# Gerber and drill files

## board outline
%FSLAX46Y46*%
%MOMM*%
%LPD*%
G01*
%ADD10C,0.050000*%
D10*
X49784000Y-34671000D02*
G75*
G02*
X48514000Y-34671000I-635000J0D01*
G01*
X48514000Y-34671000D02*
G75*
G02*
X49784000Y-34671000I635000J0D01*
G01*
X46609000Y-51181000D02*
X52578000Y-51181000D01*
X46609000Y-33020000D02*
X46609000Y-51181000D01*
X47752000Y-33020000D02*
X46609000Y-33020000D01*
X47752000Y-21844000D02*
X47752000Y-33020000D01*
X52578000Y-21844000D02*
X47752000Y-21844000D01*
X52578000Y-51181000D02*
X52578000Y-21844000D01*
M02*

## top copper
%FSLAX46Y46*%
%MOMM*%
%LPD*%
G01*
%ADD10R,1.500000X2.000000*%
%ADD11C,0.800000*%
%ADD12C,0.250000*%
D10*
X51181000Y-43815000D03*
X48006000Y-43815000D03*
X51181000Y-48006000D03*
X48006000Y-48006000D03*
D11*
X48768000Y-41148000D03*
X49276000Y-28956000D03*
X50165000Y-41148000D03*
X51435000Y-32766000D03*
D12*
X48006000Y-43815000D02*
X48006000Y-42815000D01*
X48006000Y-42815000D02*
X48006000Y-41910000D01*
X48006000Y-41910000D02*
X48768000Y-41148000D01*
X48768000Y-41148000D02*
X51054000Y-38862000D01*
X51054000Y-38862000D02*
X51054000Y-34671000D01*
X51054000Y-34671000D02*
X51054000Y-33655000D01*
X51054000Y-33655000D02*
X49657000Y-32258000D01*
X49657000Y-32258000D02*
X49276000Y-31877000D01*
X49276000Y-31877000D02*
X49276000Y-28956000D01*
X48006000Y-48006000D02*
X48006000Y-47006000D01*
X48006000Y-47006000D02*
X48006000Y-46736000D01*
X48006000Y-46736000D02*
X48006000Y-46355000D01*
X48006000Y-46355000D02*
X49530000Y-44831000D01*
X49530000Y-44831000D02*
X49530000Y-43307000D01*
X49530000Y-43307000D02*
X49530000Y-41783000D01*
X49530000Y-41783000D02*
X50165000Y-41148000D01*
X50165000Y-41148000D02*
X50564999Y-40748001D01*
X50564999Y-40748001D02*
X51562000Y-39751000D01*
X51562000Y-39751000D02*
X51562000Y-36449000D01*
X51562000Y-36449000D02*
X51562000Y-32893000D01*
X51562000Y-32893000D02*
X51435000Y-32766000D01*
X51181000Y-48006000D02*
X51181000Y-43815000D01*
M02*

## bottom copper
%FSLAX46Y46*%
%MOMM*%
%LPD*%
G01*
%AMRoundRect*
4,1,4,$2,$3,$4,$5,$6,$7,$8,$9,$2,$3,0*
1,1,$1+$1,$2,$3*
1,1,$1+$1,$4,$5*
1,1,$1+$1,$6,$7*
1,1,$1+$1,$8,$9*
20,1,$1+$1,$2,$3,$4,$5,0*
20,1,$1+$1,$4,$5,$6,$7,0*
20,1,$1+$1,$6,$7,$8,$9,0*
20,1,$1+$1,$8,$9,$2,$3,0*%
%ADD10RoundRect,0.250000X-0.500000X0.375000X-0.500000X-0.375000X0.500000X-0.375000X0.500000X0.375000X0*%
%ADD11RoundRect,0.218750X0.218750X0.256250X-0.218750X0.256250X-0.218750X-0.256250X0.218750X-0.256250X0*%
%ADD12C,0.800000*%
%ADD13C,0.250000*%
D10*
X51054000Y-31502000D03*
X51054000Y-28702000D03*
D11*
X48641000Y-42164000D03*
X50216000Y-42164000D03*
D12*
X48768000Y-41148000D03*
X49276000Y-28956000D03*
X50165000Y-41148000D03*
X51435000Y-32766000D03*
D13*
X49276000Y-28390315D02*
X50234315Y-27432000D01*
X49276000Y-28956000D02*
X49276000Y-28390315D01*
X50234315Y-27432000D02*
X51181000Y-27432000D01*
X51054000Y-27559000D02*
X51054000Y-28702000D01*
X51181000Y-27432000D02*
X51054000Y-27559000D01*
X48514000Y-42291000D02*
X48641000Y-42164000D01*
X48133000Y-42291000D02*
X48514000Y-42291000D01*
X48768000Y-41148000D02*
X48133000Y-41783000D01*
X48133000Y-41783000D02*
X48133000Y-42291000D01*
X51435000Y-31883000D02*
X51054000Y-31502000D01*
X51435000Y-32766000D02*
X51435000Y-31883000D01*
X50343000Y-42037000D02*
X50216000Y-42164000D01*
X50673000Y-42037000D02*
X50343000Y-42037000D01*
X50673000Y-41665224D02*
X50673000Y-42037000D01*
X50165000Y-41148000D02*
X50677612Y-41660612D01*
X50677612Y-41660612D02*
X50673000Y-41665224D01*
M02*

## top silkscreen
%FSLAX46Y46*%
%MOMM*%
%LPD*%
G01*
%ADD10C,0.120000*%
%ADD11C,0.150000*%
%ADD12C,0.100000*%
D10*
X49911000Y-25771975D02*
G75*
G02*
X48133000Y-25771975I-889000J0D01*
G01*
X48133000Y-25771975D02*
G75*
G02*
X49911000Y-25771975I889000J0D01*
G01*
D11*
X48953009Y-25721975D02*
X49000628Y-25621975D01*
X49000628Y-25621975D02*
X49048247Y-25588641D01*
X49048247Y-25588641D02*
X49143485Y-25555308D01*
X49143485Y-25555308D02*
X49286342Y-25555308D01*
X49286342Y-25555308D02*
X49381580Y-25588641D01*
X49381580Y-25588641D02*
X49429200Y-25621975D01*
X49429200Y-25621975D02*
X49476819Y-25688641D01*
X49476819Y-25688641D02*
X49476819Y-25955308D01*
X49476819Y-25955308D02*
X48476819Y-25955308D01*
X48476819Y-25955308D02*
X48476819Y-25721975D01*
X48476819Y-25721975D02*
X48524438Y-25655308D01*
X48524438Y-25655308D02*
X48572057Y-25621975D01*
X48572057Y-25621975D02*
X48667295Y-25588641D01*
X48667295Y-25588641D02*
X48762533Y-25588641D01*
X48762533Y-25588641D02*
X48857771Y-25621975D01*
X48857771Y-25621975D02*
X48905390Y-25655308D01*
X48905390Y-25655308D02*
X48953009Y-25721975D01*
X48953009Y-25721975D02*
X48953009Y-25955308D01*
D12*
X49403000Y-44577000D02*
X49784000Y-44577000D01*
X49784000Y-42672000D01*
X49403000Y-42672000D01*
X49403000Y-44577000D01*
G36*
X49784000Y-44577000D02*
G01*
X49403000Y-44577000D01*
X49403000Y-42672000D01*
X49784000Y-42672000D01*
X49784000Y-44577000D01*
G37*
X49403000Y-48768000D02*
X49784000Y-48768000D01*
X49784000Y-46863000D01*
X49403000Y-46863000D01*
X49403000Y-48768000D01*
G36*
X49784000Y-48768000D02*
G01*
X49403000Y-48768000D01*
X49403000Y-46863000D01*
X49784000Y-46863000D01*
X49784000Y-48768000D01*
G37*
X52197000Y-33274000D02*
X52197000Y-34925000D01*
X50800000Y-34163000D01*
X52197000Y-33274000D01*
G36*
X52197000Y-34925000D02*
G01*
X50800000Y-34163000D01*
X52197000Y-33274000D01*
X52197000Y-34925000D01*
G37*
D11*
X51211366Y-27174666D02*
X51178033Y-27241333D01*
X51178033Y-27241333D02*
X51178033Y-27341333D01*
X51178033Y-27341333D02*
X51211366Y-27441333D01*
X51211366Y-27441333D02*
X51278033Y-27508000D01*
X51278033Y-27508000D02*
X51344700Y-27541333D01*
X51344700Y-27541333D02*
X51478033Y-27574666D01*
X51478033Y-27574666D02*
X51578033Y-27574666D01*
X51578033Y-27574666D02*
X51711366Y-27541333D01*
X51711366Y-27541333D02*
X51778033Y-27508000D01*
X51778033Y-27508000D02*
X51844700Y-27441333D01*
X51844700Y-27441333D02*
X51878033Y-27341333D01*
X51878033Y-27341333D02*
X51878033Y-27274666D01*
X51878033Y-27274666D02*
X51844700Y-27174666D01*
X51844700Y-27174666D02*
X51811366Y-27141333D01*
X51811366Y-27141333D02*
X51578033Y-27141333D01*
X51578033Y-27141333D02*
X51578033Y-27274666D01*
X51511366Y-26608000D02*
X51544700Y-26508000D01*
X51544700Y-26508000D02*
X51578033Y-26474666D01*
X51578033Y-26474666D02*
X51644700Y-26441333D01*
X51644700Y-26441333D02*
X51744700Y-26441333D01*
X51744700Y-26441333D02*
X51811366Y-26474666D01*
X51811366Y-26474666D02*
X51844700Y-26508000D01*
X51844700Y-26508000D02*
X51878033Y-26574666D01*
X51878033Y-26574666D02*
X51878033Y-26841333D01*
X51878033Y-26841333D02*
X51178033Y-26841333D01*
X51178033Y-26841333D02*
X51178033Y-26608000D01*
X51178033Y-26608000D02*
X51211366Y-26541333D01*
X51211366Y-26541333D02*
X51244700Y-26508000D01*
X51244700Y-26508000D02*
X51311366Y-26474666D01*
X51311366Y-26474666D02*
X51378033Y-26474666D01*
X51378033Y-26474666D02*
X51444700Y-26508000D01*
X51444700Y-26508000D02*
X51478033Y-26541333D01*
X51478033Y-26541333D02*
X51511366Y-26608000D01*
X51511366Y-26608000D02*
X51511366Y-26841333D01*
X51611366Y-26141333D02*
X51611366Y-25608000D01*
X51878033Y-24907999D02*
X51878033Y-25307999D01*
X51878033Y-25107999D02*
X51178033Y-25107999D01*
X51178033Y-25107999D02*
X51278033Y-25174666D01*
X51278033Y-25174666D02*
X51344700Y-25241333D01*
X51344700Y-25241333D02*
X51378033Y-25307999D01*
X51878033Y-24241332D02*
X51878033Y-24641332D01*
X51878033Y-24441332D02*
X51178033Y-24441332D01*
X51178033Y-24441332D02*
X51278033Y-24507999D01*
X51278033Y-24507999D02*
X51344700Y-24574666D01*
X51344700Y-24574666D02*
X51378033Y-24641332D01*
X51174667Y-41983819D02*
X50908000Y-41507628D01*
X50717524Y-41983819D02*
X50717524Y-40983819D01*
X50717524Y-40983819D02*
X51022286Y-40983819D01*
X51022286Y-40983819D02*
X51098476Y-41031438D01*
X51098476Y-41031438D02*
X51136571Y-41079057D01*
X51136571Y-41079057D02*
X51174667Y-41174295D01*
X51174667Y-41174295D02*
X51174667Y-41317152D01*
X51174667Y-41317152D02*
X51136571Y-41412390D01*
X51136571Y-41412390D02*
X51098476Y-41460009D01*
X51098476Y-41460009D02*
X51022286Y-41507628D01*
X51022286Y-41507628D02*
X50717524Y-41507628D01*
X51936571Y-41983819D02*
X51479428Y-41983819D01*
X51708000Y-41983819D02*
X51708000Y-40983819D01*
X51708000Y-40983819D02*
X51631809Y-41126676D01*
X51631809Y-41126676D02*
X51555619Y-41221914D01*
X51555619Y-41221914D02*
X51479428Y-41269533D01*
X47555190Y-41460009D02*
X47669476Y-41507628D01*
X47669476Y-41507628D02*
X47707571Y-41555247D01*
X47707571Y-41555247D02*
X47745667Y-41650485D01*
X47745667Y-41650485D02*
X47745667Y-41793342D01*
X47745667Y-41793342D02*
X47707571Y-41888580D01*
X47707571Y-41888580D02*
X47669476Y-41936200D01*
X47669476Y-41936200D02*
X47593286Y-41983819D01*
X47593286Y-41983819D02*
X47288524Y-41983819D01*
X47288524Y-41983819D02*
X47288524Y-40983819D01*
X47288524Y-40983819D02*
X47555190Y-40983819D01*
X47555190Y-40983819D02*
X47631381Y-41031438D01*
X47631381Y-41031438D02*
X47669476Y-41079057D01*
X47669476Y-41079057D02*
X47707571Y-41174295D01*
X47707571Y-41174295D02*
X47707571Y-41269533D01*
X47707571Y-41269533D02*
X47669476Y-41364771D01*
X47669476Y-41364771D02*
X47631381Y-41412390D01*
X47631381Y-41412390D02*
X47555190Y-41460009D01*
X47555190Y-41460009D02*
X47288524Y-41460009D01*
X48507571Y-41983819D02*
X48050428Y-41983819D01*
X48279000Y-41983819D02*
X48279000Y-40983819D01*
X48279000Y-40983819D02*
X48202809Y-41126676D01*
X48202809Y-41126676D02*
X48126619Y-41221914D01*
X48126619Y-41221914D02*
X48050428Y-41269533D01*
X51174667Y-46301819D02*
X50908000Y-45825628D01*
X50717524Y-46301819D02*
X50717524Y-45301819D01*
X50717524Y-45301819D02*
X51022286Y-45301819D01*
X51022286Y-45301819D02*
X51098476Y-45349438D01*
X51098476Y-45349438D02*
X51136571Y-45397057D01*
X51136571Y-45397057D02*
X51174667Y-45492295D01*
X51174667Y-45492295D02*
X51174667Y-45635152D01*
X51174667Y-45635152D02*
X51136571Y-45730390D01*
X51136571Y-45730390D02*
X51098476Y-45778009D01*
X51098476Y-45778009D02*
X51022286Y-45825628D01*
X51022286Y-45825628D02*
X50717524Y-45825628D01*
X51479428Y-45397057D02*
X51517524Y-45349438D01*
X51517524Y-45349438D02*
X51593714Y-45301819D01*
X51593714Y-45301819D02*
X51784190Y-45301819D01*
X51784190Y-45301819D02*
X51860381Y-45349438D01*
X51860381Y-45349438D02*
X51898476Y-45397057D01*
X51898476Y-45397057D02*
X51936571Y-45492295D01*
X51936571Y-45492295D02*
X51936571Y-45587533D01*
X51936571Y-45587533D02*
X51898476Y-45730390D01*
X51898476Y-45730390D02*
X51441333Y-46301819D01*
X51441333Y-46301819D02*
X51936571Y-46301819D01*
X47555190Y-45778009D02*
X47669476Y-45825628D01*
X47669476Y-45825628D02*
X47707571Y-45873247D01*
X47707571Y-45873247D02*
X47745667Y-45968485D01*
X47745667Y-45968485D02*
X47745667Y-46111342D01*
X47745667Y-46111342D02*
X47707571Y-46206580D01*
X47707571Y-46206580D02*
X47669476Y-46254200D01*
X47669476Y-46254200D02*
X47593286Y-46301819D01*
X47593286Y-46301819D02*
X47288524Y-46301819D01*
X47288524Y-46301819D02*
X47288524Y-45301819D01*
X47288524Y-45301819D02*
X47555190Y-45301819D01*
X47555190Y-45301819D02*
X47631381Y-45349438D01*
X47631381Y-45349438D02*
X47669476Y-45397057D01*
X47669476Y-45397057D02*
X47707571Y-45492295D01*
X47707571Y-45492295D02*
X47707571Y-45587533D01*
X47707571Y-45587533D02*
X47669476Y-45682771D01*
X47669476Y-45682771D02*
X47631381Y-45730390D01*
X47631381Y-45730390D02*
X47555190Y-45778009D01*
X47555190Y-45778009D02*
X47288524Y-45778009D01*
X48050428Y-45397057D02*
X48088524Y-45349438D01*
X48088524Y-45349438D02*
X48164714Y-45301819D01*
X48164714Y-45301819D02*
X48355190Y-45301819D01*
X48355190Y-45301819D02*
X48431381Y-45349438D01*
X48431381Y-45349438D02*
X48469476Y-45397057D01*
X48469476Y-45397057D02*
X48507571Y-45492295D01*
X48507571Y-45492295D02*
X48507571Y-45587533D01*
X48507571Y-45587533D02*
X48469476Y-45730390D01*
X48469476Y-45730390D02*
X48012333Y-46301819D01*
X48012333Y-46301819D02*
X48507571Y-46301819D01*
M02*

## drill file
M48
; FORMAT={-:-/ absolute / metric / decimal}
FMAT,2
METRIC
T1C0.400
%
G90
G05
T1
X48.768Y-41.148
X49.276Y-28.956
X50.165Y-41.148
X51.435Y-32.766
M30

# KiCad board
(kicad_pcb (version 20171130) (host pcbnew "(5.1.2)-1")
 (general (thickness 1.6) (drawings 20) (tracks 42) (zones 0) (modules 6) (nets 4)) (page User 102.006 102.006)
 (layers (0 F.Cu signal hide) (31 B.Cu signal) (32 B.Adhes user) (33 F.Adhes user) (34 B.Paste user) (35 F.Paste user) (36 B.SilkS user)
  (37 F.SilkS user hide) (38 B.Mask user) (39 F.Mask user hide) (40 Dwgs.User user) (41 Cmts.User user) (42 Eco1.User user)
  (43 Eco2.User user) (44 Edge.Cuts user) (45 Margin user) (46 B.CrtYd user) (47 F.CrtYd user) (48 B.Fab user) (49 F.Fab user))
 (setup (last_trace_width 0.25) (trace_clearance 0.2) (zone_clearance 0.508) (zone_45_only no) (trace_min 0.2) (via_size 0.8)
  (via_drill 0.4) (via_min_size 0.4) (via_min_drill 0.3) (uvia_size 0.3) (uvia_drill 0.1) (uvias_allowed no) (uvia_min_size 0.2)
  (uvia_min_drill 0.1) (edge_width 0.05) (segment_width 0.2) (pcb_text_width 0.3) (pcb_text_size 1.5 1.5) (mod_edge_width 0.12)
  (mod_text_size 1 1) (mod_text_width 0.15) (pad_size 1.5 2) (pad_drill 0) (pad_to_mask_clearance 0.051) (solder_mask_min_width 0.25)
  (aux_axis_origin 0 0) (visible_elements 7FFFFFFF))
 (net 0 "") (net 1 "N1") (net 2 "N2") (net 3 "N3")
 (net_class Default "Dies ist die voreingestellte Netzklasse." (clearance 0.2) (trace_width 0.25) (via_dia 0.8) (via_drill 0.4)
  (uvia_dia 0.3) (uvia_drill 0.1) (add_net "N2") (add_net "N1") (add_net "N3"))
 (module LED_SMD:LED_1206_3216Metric (layer B.Cu) (at 51.054 30.102 270)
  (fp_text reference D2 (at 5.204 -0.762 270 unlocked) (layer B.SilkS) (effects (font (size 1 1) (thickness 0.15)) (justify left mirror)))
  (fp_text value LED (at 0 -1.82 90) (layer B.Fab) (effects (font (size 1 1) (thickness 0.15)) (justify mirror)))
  (pad 2 smd roundrect (at 1.4 0 270) (size 1.25 1.5) (layers B.Cu B.Paste B.Mask) (roundrect_rratio 0.2) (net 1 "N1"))
  (pad 1 smd roundrect (at -1.4 0 270) (size 1.25 1.5) (layers B.Cu B.Paste B.Mask) (roundrect_rratio 0.2) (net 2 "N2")))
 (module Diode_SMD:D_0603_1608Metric (layer B.Cu) (at 49.4285 42.164 180)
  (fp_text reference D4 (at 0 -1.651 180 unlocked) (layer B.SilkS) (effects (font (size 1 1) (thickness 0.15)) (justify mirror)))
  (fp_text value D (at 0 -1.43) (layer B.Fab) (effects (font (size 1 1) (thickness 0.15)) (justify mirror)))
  (pad 2 smd roundrect (at 0.7875 0 180) (size 0.875 0.95) (layers B.Cu B.Paste B.Mask) (roundrect_rratio 0.25) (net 2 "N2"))
  (pad 1 smd roundrect (at -0.7875 0 180) (size 0.875 0.95) (layers B.Cu B.Paste B.Mask) (roundrect_rratio 0.25) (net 1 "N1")))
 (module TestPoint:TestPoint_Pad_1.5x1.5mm (layer F.Cu) (at 51.181 43.815)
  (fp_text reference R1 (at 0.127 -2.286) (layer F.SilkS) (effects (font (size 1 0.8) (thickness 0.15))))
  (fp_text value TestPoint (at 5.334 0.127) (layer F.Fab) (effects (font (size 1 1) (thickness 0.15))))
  (pad 1 smd rect (at 0 0) (size 1.5 2) (layers F.Cu F.Mask) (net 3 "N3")))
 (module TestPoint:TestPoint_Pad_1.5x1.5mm (layer F.Cu) (at 48.006 43.815)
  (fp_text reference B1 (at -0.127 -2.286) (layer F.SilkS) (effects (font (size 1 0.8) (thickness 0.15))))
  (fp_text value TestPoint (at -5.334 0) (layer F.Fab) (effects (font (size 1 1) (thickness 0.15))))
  (pad 1 smd rect (at 0 0) (size 1.5 2) (layers F.Cu F.Mask) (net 2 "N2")))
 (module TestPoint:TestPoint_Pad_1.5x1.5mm (layer F.Cu) (at 51.181 48.006)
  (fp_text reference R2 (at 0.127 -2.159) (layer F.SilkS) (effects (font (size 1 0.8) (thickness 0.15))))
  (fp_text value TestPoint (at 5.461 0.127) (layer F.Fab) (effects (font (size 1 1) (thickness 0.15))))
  (pad 1 smd rect (at 0 0) (size 1.5 2) (layers F.Cu F.Mask) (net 3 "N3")))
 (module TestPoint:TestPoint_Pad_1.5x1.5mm (layer F.Cu) (at 48.006 48.006)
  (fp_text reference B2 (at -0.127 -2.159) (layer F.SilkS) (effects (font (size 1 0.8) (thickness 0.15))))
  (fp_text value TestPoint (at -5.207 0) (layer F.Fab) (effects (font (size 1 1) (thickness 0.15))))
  (pad 1 smd rect (at 0 0) (size 1.5 2) (layers F.Cu F.Mask) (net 1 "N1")))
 (gr_circle (center 49.022 25.771975) (end 49.022 24.882975) (layer F.SilkS) (width 0.12))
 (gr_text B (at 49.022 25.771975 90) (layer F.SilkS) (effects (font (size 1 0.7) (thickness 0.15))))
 (gr_poly (pts (xy 49.403 44.577) (xy 49.784 44.577) (xy 49.784 42.672) (xy 49.403 42.672)) (layer F.SilkS) (width 0.1))
 (gr_poly (pts (xy 49.403 48.768) (xy 49.784 48.768) (xy 49.784 46.863) (xy 49.403 46.863)) (layer F.SilkS) (width 0.1))
 (gr_circle (center 49.149 34.671) (end 49.149 34.036) (layer Edge.Cuts) (width 0.05))
 (gr_poly (pts (xy 52.197 33.274) (xy 52.197 34.925) (xy 50.8 34.163)) (layer F.SilkS) (width 0.1))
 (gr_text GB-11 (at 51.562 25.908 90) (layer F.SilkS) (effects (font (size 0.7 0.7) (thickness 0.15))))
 (gr_line (start 46.609 51.181) (end 52.578 51.181) (layer Edge.Cuts) (width 0.05))
 (gr_line (start 46.609 33.02) (end 46.609 51.181) (layer Edge.Cuts) (width 0.05))
 (gr_line (start 47.752 33.02) (end 46.609 33.02) (layer Edge.Cuts) (width 0.05))
 (gr_line (start 47.752 21.844) (end 47.752 33.02) (layer Edge.Cuts) (width 0.05))
 (gr_line (start 52.578 21.844) (end 47.752 21.844) (layer Edge.Cuts) (width 0.05))
 (gr_line (start 52.578 51.181) (end 52.578 21.844) (layer Edge.Cuts) (width 0.05))
 (segment (start 48.006 43.815) (end 48.006 42.815) (width 0.25) (layer F.Cu) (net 2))
 (via (at 48.768 41.148) (size 0.8) (drill 0.4) (layers F.Cu B.Cu) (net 2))
 (segment (start 48.006 42.815) (end 48.006 41.91) (width 0.25) (layer F.Cu) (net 2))
 (segment (start 48.006 41.91) (end 48.768 41.148) (width 0.25) (layer F.Cu) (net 2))
 (segment (start 48.768 41.148) (end 51.054 38.862) (width 0.25) (layer F.Cu) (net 2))
 (segment (start 51.054 38.862) (end 51.054 34.671) (width 0.25) (layer F.Cu) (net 2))
 (segment (start 51.054 34.671) (end 51.054 33.655) (width 0.25) (layer F.Cu) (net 2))
 (segment (start 51.054 33.655) (end 49.657 32.258) (width 0.25) (layer F.Cu) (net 2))
 (via (at 49.276 28.956) (size 0.8) (drill 0.4) (layers F.Cu B.Cu) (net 2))
 (segment (start 49.657 32.258) (end 49.276 31.877) (width 0.25) (layer F.Cu) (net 2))
 (segment (start 49.276 31.877) (end 49.276 28.956) (width 0.25) (layer F.Cu) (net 2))
 (segment (start 49.276 28.390315) (end 50.234315 27.432) (width 0.25) (layer B.Cu) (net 2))
 (segment (start 49.276 28.956) (end 49.276 28.390315) (width 0.25) (layer B.Cu) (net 2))
 (segment (start 50.234315 27.432) (end 51.181 27.432) (width 0.25) (layer B.Cu) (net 2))
 (segment (start 51.054 27.559) (end 51.054 28.702) (width 0.25) (layer B.Cu) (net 2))
 (segment (start 51.181 27.432) (end 51.054 27.559) (width 0.25) (layer B.Cu) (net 2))
 (segment (start 48.514 42.291) (end 48.641 42.164) (width 0.25) (layer B.Cu) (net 2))
 (segment (start 48.133 42.291) (end 48.514 42.291) (width 0.25) (layer B.Cu) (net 2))
 (segment (start 48.768 41.148) (end 48.133 41.783) (width 0.25) (layer B.Cu) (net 2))
 (segment (start 48.133 41.783) (end 48.133 42.291) (width 0.25) (layer B.Cu) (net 2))
 (segment (start 48.006 48.006) (end 48.006 47.006) (width 0.25) (layer F.Cu) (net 1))
 (segment (start 48.006 47.006) (end 48.006 46.736) (width 0.25) (layer F.Cu) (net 1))
 (segment (start 48.006 46.736) (end 48.006 46.355) (width 0.25) (layer F.Cu) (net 1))
 (segment (start 48.006 46.355) (end 49.53 44.831) (width 0.25) (layer F.Cu) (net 1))
 (segment (start 49.53 44.831) (end 49.53 43.307) (width 0.25) (layer F.Cu) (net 1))
 (via (at 50.165 41.148) (size 0.8) (drill 0.4) (layers F.Cu B.Cu) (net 1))
 (segment (start 49.53 43.307) (end 49.53 41.783) (width 0.25) (layer F.Cu) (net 1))
 (segment (start 49.53 41.783) (end 50.165 41.148) (width 0.25) (layer F.Cu) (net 1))
 (segment (start 50.165 41.148) (end 50.564999 40.748001) (width 0.25) (layer F.Cu) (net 1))
 (segment (start 50.564999 40.748001) (end 51.562 39.751) (width 0.25) (layer F.Cu) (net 1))
 (segment (start 51.562 39.751) (end 51.562 36.449) (width 0.25) (layer F.Cu) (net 1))
 (via (at 51.435 32.766) (size 0.8) (drill 0.4) (layers F.Cu B.Cu) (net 1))
 (segment (start 51.562 36.449) (end 51.562 32.893) (width 0.25) (layer F.Cu) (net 1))
 (segment (start 51.562 32.893) (end 51.435 32.766) (width 0.25) (layer F.Cu) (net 1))
 (segment (start 51.435 31.883) (end 51.054 31.502) (width 0.25) (layer B.Cu) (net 1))
 (segment (start 51.435 32.766) (end 51.435 31.883) (width 0.25) (layer B.Cu) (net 1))
 (segment (start 50.343 42.037) (end 50.216 42.164) (width 0.25) (layer B.Cu) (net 1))
 (segment (start 50.673 42.037) (end 50.343 42.037) (width 0.25) (layer B.Cu) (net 1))
 (segment (start 50.673 41.665224) (end 50.673 42.037) (width 0.25) (layer B.Cu) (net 1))
 (segment (start 50.165 41.148) (end 50.677612 41.660612) (width 0.25) (layer B.Cu) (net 1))
 (segment (start 50.677612 41.660612) (end 50.673 41.665224) (width 0.25) (layer B.Cu) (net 1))
 (segment (start 51.181 48.006) (end 51.181 43.815) (width 0.25) (layer F.Cu) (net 3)))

